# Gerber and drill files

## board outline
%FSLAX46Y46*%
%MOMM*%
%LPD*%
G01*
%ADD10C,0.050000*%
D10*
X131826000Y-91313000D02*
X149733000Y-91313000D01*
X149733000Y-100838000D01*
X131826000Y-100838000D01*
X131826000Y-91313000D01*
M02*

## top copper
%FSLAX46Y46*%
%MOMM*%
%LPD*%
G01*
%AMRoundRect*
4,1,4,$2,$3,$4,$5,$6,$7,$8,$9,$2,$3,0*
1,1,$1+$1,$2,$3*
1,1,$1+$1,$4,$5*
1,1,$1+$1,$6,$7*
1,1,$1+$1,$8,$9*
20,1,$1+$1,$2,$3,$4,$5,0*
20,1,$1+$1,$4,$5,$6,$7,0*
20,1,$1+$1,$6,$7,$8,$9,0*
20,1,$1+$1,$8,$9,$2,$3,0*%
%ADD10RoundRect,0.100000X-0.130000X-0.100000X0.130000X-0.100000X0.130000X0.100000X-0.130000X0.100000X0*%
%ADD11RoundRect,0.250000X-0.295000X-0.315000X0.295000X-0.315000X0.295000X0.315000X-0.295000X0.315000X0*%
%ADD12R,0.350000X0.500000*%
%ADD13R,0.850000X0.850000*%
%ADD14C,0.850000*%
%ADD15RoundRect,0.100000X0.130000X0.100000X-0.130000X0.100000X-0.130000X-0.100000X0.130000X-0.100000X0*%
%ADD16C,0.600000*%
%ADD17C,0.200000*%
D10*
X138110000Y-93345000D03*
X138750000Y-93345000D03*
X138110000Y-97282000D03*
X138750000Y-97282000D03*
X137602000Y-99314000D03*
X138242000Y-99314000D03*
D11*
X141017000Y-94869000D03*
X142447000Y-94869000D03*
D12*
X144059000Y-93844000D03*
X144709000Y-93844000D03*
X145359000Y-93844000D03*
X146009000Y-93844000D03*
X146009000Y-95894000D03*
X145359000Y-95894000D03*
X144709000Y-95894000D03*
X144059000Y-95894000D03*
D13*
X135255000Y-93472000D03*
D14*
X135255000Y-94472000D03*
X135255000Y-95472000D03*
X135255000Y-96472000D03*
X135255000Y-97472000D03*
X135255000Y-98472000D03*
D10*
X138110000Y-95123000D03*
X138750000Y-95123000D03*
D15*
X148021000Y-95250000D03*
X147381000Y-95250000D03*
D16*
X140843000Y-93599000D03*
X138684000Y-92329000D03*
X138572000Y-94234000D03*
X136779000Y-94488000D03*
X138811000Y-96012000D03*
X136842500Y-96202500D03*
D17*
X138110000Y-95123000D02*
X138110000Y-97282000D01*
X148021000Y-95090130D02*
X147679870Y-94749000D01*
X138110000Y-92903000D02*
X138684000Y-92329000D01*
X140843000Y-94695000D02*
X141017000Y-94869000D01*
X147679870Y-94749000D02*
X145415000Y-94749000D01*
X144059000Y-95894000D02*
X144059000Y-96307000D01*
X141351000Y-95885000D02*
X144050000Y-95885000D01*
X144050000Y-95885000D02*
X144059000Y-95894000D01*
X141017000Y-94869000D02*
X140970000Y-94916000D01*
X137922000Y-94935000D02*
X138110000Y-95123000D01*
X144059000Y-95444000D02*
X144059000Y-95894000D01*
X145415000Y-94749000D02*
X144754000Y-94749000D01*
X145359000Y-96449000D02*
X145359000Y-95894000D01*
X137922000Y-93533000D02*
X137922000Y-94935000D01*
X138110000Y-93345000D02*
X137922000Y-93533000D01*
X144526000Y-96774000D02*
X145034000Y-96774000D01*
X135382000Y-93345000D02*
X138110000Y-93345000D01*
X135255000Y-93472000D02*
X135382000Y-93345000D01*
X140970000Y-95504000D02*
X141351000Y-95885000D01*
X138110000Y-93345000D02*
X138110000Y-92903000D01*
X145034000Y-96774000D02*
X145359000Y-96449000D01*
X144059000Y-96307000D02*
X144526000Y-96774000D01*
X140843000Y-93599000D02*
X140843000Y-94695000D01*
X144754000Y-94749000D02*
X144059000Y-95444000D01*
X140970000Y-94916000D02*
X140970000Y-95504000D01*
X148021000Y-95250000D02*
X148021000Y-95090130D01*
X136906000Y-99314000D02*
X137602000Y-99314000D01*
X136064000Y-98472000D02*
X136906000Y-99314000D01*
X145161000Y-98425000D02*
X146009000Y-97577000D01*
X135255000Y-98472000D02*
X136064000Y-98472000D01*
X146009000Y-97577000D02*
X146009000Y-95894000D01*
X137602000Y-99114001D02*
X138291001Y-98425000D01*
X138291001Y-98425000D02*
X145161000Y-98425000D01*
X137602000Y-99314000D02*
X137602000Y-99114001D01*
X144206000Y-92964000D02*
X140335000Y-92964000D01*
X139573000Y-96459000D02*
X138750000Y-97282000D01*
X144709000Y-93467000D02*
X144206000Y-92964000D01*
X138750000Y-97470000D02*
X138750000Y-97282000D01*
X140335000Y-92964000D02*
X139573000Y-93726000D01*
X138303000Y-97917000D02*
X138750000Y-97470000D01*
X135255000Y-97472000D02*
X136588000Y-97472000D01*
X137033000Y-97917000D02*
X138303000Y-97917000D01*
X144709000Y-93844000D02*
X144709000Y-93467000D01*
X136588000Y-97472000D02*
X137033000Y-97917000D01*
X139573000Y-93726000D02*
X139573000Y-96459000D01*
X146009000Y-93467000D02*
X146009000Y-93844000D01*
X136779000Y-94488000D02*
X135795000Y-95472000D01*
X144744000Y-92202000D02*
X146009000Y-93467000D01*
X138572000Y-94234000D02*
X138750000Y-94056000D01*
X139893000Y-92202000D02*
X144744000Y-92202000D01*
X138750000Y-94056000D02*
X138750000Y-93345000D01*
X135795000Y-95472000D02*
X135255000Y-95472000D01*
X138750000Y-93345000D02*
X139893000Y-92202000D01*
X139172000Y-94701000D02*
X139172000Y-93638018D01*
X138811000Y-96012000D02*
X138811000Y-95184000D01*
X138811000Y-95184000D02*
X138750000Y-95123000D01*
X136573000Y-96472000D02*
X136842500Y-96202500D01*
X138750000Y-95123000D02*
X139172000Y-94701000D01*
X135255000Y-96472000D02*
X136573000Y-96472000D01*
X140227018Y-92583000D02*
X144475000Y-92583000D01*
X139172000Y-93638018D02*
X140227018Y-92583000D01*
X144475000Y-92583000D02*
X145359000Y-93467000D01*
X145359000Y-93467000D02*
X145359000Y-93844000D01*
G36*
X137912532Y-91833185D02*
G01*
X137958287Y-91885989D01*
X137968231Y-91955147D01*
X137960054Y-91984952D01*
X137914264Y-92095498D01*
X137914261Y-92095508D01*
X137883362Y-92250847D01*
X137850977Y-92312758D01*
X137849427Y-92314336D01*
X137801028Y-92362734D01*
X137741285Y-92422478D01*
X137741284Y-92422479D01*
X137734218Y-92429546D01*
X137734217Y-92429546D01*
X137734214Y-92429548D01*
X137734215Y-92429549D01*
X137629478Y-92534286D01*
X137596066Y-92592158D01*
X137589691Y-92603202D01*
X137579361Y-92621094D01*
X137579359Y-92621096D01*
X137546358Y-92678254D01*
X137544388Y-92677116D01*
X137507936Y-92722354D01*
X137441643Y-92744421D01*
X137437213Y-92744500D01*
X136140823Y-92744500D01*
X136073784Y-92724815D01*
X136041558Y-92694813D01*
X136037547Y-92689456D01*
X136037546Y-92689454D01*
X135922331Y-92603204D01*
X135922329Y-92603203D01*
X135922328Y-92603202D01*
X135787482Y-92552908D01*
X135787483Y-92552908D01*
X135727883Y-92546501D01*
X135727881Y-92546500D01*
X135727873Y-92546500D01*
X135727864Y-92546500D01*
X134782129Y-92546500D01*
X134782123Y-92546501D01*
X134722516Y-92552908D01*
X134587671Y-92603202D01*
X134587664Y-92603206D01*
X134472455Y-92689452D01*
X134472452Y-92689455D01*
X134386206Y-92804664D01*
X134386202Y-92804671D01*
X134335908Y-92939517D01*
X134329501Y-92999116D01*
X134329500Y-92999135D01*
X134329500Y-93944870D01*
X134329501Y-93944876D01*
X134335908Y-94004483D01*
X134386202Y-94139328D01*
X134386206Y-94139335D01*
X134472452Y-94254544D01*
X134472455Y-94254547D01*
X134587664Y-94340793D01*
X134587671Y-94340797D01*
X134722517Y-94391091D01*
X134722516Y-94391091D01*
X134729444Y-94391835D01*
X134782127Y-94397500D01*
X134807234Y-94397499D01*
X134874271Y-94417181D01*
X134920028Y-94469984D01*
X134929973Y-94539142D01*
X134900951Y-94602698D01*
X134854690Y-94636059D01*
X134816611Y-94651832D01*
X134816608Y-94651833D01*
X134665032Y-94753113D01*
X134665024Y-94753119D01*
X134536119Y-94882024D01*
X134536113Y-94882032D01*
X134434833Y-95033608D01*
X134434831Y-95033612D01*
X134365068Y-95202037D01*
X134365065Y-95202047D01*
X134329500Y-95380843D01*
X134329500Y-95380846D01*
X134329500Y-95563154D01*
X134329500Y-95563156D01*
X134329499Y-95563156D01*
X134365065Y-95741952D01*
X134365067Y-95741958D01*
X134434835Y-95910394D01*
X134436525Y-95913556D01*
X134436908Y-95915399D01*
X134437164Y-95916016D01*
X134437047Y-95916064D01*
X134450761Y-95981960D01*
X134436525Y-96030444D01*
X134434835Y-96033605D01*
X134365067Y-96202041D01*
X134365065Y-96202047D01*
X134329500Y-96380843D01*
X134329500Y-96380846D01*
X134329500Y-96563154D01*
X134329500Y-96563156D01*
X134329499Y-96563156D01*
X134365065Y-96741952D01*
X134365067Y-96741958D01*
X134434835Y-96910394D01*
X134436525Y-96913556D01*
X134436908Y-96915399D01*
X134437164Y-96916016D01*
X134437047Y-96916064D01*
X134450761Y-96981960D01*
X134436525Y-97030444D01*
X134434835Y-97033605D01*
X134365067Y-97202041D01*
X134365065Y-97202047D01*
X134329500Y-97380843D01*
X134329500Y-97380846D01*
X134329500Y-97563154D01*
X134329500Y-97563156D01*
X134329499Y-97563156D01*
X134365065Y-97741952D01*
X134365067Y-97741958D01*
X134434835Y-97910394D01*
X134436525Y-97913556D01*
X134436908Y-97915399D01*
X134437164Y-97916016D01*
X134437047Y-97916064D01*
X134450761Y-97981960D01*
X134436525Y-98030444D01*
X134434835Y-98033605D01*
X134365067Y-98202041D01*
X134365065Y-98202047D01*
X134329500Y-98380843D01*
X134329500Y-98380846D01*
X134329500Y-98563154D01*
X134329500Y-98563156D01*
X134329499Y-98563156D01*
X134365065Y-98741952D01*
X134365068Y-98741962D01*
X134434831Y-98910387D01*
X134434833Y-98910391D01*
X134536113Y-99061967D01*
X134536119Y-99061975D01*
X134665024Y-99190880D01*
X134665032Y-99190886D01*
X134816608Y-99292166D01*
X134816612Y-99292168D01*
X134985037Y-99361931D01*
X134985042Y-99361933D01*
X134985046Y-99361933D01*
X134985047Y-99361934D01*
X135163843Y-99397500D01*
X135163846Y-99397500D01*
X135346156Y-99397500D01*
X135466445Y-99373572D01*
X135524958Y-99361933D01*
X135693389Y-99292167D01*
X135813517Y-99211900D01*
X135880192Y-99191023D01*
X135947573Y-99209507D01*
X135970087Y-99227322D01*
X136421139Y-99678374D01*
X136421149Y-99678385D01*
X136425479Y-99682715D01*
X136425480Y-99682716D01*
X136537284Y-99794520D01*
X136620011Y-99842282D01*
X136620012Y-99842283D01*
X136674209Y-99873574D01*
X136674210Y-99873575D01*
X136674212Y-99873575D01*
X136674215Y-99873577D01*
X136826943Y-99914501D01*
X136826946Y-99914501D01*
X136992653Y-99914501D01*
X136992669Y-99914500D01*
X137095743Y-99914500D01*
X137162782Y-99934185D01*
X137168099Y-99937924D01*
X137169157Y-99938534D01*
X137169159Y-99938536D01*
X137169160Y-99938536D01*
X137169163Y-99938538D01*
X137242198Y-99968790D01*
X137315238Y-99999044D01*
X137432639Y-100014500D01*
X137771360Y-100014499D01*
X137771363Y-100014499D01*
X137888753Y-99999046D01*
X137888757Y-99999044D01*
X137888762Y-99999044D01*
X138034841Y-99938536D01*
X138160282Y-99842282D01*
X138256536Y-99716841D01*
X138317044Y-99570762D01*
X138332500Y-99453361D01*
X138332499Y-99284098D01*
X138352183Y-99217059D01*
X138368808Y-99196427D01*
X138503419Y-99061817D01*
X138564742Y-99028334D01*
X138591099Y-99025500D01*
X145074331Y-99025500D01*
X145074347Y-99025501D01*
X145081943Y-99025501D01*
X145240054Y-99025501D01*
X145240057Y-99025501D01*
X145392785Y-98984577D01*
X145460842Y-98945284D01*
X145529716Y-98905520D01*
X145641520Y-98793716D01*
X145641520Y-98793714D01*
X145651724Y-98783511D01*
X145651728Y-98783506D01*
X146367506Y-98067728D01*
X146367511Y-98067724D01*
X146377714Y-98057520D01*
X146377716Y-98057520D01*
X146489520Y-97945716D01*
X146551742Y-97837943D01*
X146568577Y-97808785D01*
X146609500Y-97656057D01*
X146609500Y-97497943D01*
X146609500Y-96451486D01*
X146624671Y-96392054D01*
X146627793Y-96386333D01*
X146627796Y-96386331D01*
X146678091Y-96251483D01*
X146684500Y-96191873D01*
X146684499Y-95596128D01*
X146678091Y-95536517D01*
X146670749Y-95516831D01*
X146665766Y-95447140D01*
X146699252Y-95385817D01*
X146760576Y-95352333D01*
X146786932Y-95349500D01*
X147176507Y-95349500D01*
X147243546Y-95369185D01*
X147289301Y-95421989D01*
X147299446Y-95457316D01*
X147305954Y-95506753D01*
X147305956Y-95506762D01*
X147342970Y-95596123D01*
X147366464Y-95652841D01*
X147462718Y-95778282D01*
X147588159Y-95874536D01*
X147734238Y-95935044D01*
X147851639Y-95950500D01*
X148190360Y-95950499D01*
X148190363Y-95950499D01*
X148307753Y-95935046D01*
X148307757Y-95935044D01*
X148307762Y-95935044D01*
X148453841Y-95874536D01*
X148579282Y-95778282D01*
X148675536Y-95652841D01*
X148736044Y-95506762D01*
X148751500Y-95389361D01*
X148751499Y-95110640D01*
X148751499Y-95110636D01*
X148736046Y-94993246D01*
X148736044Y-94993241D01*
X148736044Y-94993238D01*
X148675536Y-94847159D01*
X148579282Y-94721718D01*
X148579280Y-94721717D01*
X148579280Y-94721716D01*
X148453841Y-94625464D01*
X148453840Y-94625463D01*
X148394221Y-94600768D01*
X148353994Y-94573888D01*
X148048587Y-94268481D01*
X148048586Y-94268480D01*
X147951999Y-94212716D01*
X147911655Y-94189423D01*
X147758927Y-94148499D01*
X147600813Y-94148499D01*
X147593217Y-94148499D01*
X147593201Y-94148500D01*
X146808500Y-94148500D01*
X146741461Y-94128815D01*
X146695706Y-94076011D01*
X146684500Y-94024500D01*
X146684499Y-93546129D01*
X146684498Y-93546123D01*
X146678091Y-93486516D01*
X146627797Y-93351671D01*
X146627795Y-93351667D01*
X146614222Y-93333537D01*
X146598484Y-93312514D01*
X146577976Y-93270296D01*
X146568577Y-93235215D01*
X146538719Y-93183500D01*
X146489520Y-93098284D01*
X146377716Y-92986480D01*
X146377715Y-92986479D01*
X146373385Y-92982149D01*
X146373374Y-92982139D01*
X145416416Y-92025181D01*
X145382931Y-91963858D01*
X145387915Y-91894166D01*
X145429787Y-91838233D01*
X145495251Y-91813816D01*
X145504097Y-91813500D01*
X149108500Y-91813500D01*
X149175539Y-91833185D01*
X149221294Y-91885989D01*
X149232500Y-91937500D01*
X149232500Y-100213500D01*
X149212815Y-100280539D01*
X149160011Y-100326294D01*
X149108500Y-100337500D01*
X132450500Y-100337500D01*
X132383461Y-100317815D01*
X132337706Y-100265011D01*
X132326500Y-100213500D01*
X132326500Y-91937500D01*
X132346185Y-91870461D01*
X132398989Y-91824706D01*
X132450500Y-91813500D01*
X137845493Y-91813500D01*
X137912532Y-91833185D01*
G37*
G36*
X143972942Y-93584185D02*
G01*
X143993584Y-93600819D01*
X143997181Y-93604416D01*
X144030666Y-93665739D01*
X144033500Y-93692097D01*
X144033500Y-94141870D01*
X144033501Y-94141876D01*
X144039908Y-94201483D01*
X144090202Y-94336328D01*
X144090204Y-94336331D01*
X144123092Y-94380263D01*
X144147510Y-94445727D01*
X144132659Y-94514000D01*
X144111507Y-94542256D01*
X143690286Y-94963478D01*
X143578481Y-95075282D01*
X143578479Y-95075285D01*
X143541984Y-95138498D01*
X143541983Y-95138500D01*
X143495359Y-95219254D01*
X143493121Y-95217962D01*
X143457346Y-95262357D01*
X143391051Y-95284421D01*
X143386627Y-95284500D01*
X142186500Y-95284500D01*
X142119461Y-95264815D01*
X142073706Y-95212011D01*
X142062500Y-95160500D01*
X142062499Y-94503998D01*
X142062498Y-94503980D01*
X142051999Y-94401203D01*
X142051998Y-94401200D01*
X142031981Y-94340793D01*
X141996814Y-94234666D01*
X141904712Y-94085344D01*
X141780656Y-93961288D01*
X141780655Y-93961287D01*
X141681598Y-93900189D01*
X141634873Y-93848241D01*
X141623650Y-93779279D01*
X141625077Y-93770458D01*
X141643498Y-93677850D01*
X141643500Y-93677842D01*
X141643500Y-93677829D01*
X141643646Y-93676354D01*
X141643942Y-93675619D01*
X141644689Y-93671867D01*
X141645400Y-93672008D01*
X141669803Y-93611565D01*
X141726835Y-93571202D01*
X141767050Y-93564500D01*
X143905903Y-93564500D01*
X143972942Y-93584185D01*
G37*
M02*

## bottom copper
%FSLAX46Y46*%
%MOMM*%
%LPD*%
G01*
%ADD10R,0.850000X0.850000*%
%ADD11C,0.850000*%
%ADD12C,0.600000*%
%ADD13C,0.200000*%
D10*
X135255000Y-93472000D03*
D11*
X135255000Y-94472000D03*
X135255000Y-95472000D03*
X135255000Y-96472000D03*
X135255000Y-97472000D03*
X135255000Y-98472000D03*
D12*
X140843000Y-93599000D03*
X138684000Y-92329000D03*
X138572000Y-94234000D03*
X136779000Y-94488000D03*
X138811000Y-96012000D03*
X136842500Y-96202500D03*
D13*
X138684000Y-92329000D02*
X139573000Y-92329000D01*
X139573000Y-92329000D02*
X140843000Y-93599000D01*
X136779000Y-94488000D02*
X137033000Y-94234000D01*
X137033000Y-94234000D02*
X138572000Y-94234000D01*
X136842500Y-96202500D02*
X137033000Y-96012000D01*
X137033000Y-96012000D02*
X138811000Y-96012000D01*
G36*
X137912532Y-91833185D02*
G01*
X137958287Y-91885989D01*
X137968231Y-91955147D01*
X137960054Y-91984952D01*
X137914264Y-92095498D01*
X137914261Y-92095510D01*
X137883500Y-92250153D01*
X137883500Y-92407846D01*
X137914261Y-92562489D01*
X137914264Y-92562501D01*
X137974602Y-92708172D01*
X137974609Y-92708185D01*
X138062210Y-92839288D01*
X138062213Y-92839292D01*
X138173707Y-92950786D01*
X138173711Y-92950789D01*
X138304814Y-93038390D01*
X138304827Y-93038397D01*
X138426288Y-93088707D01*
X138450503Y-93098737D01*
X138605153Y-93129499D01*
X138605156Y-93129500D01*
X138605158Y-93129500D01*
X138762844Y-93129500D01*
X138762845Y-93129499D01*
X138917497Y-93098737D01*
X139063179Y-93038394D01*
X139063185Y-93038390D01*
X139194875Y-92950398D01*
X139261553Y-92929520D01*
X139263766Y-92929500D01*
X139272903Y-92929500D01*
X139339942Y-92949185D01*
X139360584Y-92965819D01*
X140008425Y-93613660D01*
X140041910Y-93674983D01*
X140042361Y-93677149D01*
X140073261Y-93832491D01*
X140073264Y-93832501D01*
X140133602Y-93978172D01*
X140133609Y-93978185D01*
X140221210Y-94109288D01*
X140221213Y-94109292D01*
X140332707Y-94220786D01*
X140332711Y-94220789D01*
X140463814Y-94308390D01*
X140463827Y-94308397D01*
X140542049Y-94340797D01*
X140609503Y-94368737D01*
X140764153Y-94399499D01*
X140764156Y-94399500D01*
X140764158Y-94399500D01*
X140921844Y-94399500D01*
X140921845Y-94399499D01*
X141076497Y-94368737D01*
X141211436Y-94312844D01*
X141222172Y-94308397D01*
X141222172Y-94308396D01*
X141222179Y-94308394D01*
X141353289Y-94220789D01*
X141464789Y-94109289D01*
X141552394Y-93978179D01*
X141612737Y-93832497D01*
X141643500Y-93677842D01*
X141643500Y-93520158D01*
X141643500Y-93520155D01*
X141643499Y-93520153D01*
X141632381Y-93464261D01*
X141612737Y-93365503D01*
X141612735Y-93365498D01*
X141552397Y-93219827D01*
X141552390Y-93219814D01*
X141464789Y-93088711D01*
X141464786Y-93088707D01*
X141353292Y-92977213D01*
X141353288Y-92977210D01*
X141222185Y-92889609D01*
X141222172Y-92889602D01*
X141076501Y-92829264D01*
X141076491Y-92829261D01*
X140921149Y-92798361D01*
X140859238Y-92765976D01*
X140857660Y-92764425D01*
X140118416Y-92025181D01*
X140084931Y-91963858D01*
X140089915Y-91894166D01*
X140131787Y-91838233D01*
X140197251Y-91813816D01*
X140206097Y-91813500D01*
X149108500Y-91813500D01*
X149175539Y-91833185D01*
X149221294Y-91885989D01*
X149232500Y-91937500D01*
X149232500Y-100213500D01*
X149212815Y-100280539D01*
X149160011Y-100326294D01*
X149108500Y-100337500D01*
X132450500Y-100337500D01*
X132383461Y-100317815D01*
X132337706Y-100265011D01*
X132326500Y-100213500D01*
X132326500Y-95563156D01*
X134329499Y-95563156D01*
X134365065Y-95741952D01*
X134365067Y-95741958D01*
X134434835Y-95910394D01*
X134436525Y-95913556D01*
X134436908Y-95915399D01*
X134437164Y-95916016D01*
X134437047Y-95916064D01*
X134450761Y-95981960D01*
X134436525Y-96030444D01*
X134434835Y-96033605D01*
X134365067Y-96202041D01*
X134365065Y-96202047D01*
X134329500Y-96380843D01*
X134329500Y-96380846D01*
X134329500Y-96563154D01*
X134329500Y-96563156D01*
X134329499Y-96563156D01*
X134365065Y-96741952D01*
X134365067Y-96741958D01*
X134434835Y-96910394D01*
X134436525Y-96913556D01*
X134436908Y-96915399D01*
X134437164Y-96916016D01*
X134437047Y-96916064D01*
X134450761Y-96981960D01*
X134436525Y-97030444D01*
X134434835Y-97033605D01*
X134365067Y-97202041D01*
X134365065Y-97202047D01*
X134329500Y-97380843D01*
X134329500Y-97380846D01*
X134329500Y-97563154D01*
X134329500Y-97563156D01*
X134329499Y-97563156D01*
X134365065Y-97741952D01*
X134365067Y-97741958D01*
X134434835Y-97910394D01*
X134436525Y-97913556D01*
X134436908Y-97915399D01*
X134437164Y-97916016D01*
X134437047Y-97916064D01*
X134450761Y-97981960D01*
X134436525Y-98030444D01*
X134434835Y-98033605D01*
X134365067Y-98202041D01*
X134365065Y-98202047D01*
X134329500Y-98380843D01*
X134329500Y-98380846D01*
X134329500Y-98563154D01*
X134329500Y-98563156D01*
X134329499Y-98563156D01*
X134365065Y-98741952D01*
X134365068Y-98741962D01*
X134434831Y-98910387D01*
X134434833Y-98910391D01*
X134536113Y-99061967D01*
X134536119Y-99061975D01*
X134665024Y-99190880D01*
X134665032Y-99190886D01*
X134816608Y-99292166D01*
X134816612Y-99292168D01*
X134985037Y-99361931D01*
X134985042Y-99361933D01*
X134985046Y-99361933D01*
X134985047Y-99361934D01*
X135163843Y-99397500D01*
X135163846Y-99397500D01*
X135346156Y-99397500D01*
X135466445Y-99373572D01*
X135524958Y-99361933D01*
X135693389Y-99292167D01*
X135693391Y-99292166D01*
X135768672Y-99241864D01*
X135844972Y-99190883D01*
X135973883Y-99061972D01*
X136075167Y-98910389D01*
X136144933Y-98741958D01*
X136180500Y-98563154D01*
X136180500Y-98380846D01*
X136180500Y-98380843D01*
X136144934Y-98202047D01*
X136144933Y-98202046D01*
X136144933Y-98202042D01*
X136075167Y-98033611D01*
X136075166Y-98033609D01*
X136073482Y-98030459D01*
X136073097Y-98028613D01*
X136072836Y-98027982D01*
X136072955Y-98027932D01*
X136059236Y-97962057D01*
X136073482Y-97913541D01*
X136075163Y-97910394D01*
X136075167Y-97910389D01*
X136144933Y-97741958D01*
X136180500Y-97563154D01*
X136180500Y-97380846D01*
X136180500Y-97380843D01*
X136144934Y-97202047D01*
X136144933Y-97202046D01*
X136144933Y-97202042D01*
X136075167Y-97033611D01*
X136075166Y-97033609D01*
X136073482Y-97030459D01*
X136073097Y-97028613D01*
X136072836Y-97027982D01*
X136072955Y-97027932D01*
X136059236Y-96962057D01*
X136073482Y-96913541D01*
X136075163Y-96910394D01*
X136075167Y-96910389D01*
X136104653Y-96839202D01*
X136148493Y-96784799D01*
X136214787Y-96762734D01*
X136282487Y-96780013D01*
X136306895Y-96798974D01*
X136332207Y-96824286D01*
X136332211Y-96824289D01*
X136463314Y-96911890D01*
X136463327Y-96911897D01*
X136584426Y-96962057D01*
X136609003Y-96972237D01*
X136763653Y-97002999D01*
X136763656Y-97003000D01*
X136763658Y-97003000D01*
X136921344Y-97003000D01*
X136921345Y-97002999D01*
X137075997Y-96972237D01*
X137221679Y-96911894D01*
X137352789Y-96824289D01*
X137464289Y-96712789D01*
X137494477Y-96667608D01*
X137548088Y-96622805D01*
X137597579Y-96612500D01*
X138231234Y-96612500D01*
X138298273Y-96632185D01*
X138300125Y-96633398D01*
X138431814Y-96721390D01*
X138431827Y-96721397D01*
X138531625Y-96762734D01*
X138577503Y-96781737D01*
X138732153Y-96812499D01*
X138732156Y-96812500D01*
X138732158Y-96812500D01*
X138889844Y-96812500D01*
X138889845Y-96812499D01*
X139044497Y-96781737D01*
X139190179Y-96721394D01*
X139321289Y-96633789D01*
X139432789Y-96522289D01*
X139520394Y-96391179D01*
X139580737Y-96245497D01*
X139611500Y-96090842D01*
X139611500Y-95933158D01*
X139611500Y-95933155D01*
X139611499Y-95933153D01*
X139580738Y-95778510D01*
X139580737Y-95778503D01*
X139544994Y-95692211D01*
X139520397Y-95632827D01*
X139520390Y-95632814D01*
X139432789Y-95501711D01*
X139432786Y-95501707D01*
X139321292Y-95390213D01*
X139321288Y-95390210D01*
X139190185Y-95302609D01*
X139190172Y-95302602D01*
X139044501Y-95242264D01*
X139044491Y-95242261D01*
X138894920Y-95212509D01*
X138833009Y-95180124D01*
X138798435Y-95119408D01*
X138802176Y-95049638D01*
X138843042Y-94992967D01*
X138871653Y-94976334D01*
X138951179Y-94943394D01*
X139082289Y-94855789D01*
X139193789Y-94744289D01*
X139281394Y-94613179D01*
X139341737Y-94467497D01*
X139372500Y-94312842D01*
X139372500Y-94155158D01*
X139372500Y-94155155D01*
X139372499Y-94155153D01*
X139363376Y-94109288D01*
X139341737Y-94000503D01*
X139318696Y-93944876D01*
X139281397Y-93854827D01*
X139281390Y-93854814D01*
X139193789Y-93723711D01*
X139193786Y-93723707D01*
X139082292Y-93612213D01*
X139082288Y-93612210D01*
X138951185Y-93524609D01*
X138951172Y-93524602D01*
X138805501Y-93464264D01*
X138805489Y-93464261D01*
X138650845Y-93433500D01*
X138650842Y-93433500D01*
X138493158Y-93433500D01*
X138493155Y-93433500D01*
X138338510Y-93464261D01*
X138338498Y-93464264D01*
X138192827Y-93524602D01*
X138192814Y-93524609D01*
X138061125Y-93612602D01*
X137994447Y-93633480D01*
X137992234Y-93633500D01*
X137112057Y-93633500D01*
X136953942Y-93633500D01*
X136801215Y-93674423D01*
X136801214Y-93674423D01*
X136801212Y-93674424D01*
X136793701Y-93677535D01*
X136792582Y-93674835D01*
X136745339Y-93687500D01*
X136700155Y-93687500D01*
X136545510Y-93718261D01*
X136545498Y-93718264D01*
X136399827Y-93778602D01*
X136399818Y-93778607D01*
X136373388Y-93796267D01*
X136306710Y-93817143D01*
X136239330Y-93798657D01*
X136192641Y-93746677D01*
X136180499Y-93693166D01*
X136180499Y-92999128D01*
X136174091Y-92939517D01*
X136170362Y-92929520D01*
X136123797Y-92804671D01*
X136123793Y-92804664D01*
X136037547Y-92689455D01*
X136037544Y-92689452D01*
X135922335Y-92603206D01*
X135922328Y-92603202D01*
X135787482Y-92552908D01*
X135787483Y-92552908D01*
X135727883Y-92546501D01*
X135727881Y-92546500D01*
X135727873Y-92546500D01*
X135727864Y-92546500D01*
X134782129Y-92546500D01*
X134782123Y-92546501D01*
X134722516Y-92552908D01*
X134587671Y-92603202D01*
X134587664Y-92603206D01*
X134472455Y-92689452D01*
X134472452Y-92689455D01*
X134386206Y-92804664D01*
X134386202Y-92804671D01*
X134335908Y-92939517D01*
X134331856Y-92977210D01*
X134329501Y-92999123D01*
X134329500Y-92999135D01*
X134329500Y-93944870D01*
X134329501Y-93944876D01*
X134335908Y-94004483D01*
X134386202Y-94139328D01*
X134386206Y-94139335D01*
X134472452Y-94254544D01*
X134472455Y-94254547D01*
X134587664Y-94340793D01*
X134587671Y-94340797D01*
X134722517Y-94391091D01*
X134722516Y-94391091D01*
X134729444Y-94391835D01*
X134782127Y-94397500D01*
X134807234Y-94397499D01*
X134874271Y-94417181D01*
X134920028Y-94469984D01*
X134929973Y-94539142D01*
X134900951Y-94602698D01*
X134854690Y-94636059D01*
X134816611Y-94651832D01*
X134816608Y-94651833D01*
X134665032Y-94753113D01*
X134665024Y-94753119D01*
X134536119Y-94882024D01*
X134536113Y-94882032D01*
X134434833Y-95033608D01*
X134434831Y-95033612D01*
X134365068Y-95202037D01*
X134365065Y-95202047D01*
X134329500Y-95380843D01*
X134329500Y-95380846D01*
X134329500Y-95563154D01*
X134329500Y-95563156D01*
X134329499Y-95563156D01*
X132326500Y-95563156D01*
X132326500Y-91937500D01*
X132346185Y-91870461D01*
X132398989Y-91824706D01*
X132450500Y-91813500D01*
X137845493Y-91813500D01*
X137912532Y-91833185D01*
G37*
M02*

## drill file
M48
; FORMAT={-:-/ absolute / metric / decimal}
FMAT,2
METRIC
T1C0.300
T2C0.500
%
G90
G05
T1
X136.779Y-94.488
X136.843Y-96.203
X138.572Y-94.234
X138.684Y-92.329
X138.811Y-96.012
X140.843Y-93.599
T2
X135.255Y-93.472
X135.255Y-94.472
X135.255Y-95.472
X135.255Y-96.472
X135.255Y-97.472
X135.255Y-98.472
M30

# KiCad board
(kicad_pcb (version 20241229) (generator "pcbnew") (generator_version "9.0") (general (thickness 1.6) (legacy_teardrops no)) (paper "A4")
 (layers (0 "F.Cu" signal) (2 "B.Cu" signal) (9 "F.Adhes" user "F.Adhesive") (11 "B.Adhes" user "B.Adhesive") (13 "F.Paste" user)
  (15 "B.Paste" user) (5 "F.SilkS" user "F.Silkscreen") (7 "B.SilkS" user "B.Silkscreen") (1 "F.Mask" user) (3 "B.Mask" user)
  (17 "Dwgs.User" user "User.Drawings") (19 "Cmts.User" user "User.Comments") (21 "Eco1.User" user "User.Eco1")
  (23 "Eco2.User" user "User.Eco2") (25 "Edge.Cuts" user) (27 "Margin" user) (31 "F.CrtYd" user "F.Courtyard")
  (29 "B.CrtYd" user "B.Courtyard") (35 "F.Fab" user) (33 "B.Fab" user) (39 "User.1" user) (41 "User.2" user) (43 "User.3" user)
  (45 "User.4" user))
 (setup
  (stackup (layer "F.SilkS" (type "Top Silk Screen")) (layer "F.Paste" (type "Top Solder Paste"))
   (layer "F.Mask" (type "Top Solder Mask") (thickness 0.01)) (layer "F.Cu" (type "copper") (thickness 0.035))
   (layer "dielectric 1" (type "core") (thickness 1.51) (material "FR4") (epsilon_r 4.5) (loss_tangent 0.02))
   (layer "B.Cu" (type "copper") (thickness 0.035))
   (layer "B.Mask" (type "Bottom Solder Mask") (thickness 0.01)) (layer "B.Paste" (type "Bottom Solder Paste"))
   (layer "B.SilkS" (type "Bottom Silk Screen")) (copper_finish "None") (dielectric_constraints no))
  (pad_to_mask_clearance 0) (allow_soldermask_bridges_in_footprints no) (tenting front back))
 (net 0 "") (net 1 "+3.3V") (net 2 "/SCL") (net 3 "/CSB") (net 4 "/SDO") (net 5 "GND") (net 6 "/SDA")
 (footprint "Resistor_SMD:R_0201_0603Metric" (layer "F.Cu") (at 138.43 93.345)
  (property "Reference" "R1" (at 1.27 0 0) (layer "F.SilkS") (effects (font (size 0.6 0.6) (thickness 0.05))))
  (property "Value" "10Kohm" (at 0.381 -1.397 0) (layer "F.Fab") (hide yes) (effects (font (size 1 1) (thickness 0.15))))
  (pad "" smd roundrect (at -0.345 0) (size 0.318 0.36) (layers "F.Paste") (roundrect_rratio 0.25))
  (pad "" smd roundrect (at 0.345 0) (size 0.318 0.36) (layers "F.Paste") (roundrect_rratio 0.25))
  (pad "1" smd roundrect (at -0.32 0) (size 0.46 0.4) (layers "F.Cu" "F.Mask") (roundrect_rratio 0.25) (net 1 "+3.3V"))
  (pad "2" smd roundrect (at 0.32 0) (size 0.46 0.4) (layers "F.Cu" "F.Mask") (roundrect_rratio 0.25) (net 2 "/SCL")))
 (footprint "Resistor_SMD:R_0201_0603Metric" (layer "F.Cu") (at 138.43 97.282)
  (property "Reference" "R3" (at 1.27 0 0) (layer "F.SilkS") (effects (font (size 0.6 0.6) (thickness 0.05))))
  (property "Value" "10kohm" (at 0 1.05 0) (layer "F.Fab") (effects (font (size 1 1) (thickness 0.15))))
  (pad "" smd roundrect (at -0.345 0) (size 0.318 0.36) (layers "F.Paste") (roundrect_rratio 0.25))
  (pad "" smd roundrect (at 0.345 0) (size 0.318 0.36) (layers "F.Paste") (roundrect_rratio 0.25))
  (pad "1" smd roundrect (at -0.32 0) (size 0.46 0.4) (layers "F.Cu" "F.Mask") (roundrect_rratio 0.25) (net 1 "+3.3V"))
  (pad "2" smd roundrect (at 0.32 0) (size 0.46 0.4) (layers "F.Cu" "F.Mask") (roundrect_rratio 0.25) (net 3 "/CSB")))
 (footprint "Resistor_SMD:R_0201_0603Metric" (layer "F.Cu") (at 137.922 99.314)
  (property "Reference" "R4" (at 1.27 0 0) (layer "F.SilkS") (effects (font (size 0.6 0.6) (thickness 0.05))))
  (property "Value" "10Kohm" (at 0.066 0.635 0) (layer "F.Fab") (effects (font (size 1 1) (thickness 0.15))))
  (pad "" smd roundrect (at -0.345 0) (size 0.318 0.36) (layers "F.Paste") (roundrect_rratio 0.25))
  (pad "" smd roundrect (at 0.345 0) (size 0.318 0.36) (layers "F.Paste") (roundrect_rratio 0.25))
  (pad "1" smd roundrect (at -0.32 0) (size 0.46 0.4) (layers "F.Cu" "F.Mask") (roundrect_rratio 0.25) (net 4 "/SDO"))
  (pad "2" smd roundrect (at 0.32 0) (size 0.46 0.4) (layers "F.Cu" "F.Mask") (roundrect_rratio 0.25) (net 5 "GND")))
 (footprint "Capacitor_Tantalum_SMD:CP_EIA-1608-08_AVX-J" (layer "F.Cu") (at 141.732 94.869)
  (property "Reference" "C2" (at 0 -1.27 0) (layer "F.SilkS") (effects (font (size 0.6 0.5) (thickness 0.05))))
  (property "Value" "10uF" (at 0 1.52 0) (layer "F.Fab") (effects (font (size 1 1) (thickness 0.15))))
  (pad "1" smd roundrect (at -0.715 0) (size 1.09 1.13) (layers "F.Cu" "F.Mask" "F.Paste") (roundrect_rratio 0.229358) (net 1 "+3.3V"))
  (pad "2" smd roundrect (at 0.715 0) (size 1.09 1.13) (layers "F.Cu" "F.Mask" "F.Paste") (roundrect_rratio 0.229358) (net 5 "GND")))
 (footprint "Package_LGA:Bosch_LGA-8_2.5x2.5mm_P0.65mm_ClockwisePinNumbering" (layer "F.Cu") (at 145.034 94.869)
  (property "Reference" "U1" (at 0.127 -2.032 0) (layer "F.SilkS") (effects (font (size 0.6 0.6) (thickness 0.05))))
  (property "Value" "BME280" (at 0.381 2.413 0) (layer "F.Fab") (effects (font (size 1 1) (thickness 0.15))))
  (pad "1" smd rect (at -0.975 -1.025 90) (size 0.5 0.35) (layers "F.Cu" "F.Mask" "F.Paste") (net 5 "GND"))
  (pad "2" smd rect (at -0.325 -1.025 90) (size 0.5 0.35) (layers "F.Cu" "F.Mask" "F.Paste") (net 3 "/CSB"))
  (pad "3" smd rect (at 0.325 -1.025 90) (size 0.5 0.35) (layers "F.Cu" "F.Mask" "F.Paste") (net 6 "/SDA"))
  (pad "4" smd rect (at 0.975 -1.025 90) (size 0.5 0.35) (layers "F.Cu" "F.Mask" "F.Paste") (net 2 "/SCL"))
  (pad "5" smd rect (at 0.975 1.025 90) (size 0.5 0.35) (layers "F.Cu" "F.Mask" "F.Paste") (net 4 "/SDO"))
  (pad "6" smd rect (at 0.325 1.025 90) (size 0.5 0.35) (layers "F.Cu" "F.Mask" "F.Paste") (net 1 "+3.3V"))
  (pad "7" smd rect (at -0.325 1.025 90) (size 0.5 0.35) (layers "F.Cu" "F.Mask" "F.Paste") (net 5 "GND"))
  (pad "8" smd rect (at -0.975 1.025 90) (size 0.5 0.35) (layers "F.Cu" "F.Mask" "F.Paste") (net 1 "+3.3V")))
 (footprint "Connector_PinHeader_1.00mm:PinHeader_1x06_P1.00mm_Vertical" (layer "F.Cu") (at 135.255 93.472)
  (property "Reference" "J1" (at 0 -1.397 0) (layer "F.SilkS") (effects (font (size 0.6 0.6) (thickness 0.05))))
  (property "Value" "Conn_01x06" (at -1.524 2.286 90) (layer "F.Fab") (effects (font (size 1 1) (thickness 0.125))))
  (pad "1" thru_hole rect (at 0 0) (size 0.85 0.85) (drill 0.5) (layers "*.Cu" "*.Mask") (remove_unused_layers no) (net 1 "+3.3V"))
  (pad "2" thru_hole circle (at 0 1) (size 0.85 0.85) (drill 0.5) (layers "*.Cu" "*.Mask") (remove_unused_layers no) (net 5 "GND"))
  (pad "3" thru_hole circle (at 0 2) (size 0.85 0.85) (drill 0.5) (layers "*.Cu" "*.Mask") (remove_unused_layers no) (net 2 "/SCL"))
  (pad "4" thru_hole circle (at 0 3) (size 0.85 0.85) (drill 0.5) (layers "*.Cu" "*.Mask") (remove_unused_layers no) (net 6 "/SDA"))
  (pad "5" thru_hole circle (at 0 4) (size 0.85 0.85) (drill 0.5) (layers "*.Cu" "*.Mask") (remove_unused_layers no) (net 3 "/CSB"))
  (pad "6" thru_hole circle (at 0 5) (size 0.85 0.85) (drill 0.5) (layers "*.Cu" "*.Mask") (remove_unused_layers no) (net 4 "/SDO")))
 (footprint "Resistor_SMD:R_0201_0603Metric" (layer "F.Cu") (at 138.43 95.123)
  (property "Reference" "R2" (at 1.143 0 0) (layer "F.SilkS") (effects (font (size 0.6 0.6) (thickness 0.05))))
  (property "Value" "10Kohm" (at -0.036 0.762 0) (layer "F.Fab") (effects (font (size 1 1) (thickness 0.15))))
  (pad "" smd roundrect (at -0.345 0) (size 0.318 0.36) (layers "F.Paste") (roundrect_rratio 0.25))
  (pad "" smd roundrect (at 0.345 0) (size 0.318 0.36) (layers "F.Paste") (roundrect_rratio 0.25))
  (pad "1" smd roundrect (at -0.32 0) (size 0.46 0.4) (layers "F.Cu" "F.Mask") (roundrect_rratio 0.25) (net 1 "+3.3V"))
  (pad "2" smd roundrect (at 0.32 0) (size 0.46 0.4) (layers "F.Cu" "F.Mask") (roundrect_rratio 0.25) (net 6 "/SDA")))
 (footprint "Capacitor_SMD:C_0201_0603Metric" (layer "F.Cu") (at 147.701 95.25 180)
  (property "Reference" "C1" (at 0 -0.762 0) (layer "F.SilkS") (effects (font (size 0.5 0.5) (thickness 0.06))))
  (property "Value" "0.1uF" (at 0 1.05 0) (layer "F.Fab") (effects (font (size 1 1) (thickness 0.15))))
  (pad "" smd roundrect (at -0.345 0 180) (size 0.318 0.36) (layers "F.Paste") (roundrect_rratio 0.25))
  (pad "" smd roundrect (at 0.345 0 180) (size 0.318 0.36) (layers "F.Paste") (roundrect_rratio 0.25))
  (pad "1" smd roundrect (at -0.32 0 180) (size 0.46 0.4) (layers "F.Cu" "F.Mask") (roundrect_rratio 0.25) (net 1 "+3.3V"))
  (pad "2" smd roundrect (at 0.32 0 180) (size 0.46 0.4) (layers "F.Cu" "F.Mask") (roundrect_rratio 0.25) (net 5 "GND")))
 (gr_rect (start 131.826 91.313) (end 149.733 100.838) (stroke (width 0.05) (type default)) (fill no) (layer "Edge.Cuts"))
 (segment (start 138.11 95.123) (end 138.11 97.282) (width 0.2) (layer "F.Cu") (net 1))
 (segment (start 148.021 95.09013) (end 147.67987 94.749) (width 0.2) (layer "F.Cu") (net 1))
 (segment (start 138.11 92.903) (end 138.684 92.329) (width 0.2) (layer "F.Cu") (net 1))
 (segment (start 140.843 94.695) (end 141.017 94.869) (width 0.2) (layer "F.Cu") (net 1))
 (segment (start 147.67987 94.749) (end 145.415 94.749) (width 0.2) (layer "F.Cu") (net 1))
 (segment (start 144.059 95.894) (end 144.059 96.307) (width 0.2) (layer "F.Cu") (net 1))
 (segment (start 141.351 95.885) (end 144.05 95.885) (width 0.2) (layer "F.Cu") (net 1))
 (segment (start 144.05 95.885) (end 144.059 95.894) (width 0.2) (layer "F.Cu") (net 1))
 (segment (start 141.017 94.869) (end 140.97 94.916) (width 0.2) (layer "F.Cu") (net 1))
 (segment (start 137.922 94.935) (end 138.11 95.123) (width 0.2) (layer "F.Cu") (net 1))
 (segment (start 144.059 95.444) (end 144.059 95.894) (width 0.2) (layer "F.Cu") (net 1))
 (segment (start 145.415 94.749) (end 144.754 94.749) (width 0.2) (layer "F.Cu") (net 1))
 (segment (start 145.359 96.449) (end 145.359 95.894) (width 0.2) (layer "F.Cu") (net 1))
 (segment (start 137.922 93.533) (end 137.922 94.935) (width 0.2) (layer "F.Cu") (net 1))
 (segment (start 138.11 93.345) (end 137.922 93.533) (width 0.2) (layer "F.Cu") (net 1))
 (segment (start 144.526 96.774) (end 145.034 96.774) (width 0.2) (layer "F.Cu") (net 1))
 (segment (start 135.382 93.345) (end 138.11 93.345) (width 0.2) (layer "F.Cu") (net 1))
 (segment (start 135.255 93.472) (end 135.382 93.345) (width 0.2) (layer "F.Cu") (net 1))
 (segment (start 140.97 95.504) (end 141.351 95.885) (width 0.2) (layer "F.Cu") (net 1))
 (segment (start 138.11 93.345) (end 138.11 92.903) (width 0.2) (layer "F.Cu") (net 1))
 (segment (start 145.034 96.774) (end 145.359 96.449) (width 0.2) (layer "F.Cu") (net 1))
 (segment (start 144.059 96.307) (end 144.526 96.774) (width 0.2) (layer "F.Cu") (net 1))
 (segment (start 140.843 93.599) (end 140.843 94.695) (width 0.2) (layer "F.Cu") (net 1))
 (segment (start 144.754 94.749) (end 144.059 95.444) (width 0.2) (layer "F.Cu") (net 1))
 (segment (start 140.97 94.916) (end 140.97 95.504) (width 0.2) (layer "F.Cu") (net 1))
 (segment (start 148.021 95.25) (end 148.021 95.09013) (width 0.2) (layer "F.Cu") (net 1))
 (via (at 140.843 93.599) (size 0.6) (drill 0.3) (layers "F.Cu" "B.Cu") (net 1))
 (via (at 138.684 92.329) (size 0.6) (drill 0.3) (layers "F.Cu" "B.Cu") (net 1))
 (segment (start 138.684 92.329) (end 139.573 92.329) (width 0.2) (layer "B.Cu") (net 1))
 (segment (start 139.573 92.329) (end 140.843 93.599) (width 0.2) (layer "B.Cu") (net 1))
 (segment (start 136.906 99.314) (end 137.602 99.314) (width 0.2) (layer "F.Cu") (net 4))
 (segment (start 136.064 98.472) (end 136.906 99.314) (width 0.2) (layer "F.Cu") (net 4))
 (segment (start 145.161 98.425) (end 146.009 97.577) (width 0.2) (layer "F.Cu") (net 4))
 (segment (start 135.255 98.472) (end 136.064 98.472) (width 0.2) (layer "F.Cu") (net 4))
 (segment (start 146.009 97.577) (end 146.009 95.894) (width 0.2) (layer "F.Cu") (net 4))
 (segment (start 137.602 99.114001) (end 138.291001 98.425) (width 0.2) (layer "F.Cu") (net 4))
 (segment (start 138.291001 98.425) (end 145.161 98.425) (width 0.2) (layer "F.Cu") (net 4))
 (segment (start 137.602 99.314) (end 137.602 99.114001) (width 0.2) (layer "F.Cu") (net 4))
 (segment (start 144.206 92.964) (end 140.335 92.964) (width 0.2) (layer "F.Cu") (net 3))
 (segment (start 139.573 96.459) (end 138.75 97.282) (width 0.2) (layer "F.Cu") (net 3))
 (segment (start 144.709 93.467) (end 144.206 92.964) (width 0.2) (layer "F.Cu") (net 3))
 (segment (start 138.75 97.47) (end 138.75 97.282) (width 0.2) (layer "F.Cu") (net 3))
 (segment (start 140.335 92.964) (end 139.573 93.726) (width 0.2) (layer "F.Cu") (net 3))
 (segment (start 138.303 97.917) (end 138.75 97.47) (width 0.2) (layer "F.Cu") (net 3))
 (segment (start 135.255 97.472) (end 136.588 97.472) (width 0.2) (layer "F.Cu") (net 3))
 (segment (start 137.033 97.917) (end 138.303 97.917) (width 0.2) (layer "F.Cu") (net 3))
 (segment (start 144.709 93.844) (end 144.709 93.467) (width 0.2) (layer "F.Cu") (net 3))
 (segment (start 136.588 97.472) (end 137.033 97.917) (width 0.2) (layer "F.Cu") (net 3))
 (segment (start 139.573 93.726) (end 139.573 96.459) (width 0.2) (layer "F.Cu") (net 3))
 (segment (start 146.009 93.467) (end 146.009 93.844) (width 0.2) (layer "F.Cu") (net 2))
 (segment (start 136.779 94.488) (end 135.795 95.472) (width 0.2) (layer "F.Cu") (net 2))
 (segment (start 144.744 92.202) (end 146.009 93.467) (width 0.2) (layer "F.Cu") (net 2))
 (segment (start 138.572 94.234) (end 138.75 94.056) (width 0.2) (layer "F.Cu") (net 2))
 (segment (start 139.893 92.202) (end 144.744 92.202) (width 0.2) (layer "F.Cu") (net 2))
 (segment (start 138.75 94.056) (end 138.75 93.345) (width 0.2) (layer "F.Cu") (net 2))
 (segment (start 135.795 95.472) (end 135.255 95.472) (width 0.2) (layer "F.Cu") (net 2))
 (segment (start 138.75 93.345) (end 139.893 92.202) (width 0.2) (layer "F.Cu") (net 2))
 (via (at 138.572 94.234) (size 0.6) (drill 0.3) (layers "F.Cu" "B.Cu") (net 2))
 (via (at 136.779 94.488) (size 0.6) (drill 0.3) (layers "F.Cu" "B.Cu") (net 2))
 (segment (start 136.779 94.488) (end 137.033 94.234) (width 0.2) (layer "B.Cu") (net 2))
 (segment (start 137.033 94.234) (end 138.572 94.234) (width 0.2) (layer "B.Cu") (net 2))
 (segment (start 139.172 94.701) (end 139.172 93.638018) (width 0.2) (layer "F.Cu") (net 6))
 (segment (start 138.811 96.012) (end 138.811 95.184) (width 0.2) (layer "F.Cu") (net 6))
 (segment (start 138.811 95.184) (end 138.75 95.123) (width 0.2) (layer "F.Cu") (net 6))
 (segment (start 136.573 96.472) (end 136.8425 96.2025) (width 0.2) (layer "F.Cu") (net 6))
 (segment (start 138.75 95.123) (end 139.172 94.701) (width 0.2) (layer "F.Cu") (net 6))
 (segment (start 135.255 96.472) (end 136.573 96.472) (width 0.2) (layer "F.Cu") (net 6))
 (segment (start 140.227018 92.583) (end 144.475 92.583) (width 0.2) (layer "F.Cu") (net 6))
 (segment (start 139.172 93.638018) (end 140.227018 92.583) (width 0.2) (layer "F.Cu") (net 6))
 (segment (start 144.475 92.583) (end 145.359 93.467) (width 0.2) (layer "F.Cu") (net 6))
 (segment (start 145.359 93.467) (end 145.359 93.844) (width 0.2) (layer "F.Cu") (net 6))
 (via (at 138.811 96.012) (size 0.6) (drill 0.3) (layers "F.Cu" "B.Cu") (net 6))
 (via (at 136.8425 96.2025) (size 0.6) (drill 0.3) (layers "F.Cu" "B.Cu") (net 6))
 (segment (start 136.8425 96.2025) (end 137.033 96.012) (width 0.2) (layer "B.Cu") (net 6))
 (segment (start 137.033 96.012) (end 138.811 96.012) (width 0.2) (layer "B.Cu") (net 6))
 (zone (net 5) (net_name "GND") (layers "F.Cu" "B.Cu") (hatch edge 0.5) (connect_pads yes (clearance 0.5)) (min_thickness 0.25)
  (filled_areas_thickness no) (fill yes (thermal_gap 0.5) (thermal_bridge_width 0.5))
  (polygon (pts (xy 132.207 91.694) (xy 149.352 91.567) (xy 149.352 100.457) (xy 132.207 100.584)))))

